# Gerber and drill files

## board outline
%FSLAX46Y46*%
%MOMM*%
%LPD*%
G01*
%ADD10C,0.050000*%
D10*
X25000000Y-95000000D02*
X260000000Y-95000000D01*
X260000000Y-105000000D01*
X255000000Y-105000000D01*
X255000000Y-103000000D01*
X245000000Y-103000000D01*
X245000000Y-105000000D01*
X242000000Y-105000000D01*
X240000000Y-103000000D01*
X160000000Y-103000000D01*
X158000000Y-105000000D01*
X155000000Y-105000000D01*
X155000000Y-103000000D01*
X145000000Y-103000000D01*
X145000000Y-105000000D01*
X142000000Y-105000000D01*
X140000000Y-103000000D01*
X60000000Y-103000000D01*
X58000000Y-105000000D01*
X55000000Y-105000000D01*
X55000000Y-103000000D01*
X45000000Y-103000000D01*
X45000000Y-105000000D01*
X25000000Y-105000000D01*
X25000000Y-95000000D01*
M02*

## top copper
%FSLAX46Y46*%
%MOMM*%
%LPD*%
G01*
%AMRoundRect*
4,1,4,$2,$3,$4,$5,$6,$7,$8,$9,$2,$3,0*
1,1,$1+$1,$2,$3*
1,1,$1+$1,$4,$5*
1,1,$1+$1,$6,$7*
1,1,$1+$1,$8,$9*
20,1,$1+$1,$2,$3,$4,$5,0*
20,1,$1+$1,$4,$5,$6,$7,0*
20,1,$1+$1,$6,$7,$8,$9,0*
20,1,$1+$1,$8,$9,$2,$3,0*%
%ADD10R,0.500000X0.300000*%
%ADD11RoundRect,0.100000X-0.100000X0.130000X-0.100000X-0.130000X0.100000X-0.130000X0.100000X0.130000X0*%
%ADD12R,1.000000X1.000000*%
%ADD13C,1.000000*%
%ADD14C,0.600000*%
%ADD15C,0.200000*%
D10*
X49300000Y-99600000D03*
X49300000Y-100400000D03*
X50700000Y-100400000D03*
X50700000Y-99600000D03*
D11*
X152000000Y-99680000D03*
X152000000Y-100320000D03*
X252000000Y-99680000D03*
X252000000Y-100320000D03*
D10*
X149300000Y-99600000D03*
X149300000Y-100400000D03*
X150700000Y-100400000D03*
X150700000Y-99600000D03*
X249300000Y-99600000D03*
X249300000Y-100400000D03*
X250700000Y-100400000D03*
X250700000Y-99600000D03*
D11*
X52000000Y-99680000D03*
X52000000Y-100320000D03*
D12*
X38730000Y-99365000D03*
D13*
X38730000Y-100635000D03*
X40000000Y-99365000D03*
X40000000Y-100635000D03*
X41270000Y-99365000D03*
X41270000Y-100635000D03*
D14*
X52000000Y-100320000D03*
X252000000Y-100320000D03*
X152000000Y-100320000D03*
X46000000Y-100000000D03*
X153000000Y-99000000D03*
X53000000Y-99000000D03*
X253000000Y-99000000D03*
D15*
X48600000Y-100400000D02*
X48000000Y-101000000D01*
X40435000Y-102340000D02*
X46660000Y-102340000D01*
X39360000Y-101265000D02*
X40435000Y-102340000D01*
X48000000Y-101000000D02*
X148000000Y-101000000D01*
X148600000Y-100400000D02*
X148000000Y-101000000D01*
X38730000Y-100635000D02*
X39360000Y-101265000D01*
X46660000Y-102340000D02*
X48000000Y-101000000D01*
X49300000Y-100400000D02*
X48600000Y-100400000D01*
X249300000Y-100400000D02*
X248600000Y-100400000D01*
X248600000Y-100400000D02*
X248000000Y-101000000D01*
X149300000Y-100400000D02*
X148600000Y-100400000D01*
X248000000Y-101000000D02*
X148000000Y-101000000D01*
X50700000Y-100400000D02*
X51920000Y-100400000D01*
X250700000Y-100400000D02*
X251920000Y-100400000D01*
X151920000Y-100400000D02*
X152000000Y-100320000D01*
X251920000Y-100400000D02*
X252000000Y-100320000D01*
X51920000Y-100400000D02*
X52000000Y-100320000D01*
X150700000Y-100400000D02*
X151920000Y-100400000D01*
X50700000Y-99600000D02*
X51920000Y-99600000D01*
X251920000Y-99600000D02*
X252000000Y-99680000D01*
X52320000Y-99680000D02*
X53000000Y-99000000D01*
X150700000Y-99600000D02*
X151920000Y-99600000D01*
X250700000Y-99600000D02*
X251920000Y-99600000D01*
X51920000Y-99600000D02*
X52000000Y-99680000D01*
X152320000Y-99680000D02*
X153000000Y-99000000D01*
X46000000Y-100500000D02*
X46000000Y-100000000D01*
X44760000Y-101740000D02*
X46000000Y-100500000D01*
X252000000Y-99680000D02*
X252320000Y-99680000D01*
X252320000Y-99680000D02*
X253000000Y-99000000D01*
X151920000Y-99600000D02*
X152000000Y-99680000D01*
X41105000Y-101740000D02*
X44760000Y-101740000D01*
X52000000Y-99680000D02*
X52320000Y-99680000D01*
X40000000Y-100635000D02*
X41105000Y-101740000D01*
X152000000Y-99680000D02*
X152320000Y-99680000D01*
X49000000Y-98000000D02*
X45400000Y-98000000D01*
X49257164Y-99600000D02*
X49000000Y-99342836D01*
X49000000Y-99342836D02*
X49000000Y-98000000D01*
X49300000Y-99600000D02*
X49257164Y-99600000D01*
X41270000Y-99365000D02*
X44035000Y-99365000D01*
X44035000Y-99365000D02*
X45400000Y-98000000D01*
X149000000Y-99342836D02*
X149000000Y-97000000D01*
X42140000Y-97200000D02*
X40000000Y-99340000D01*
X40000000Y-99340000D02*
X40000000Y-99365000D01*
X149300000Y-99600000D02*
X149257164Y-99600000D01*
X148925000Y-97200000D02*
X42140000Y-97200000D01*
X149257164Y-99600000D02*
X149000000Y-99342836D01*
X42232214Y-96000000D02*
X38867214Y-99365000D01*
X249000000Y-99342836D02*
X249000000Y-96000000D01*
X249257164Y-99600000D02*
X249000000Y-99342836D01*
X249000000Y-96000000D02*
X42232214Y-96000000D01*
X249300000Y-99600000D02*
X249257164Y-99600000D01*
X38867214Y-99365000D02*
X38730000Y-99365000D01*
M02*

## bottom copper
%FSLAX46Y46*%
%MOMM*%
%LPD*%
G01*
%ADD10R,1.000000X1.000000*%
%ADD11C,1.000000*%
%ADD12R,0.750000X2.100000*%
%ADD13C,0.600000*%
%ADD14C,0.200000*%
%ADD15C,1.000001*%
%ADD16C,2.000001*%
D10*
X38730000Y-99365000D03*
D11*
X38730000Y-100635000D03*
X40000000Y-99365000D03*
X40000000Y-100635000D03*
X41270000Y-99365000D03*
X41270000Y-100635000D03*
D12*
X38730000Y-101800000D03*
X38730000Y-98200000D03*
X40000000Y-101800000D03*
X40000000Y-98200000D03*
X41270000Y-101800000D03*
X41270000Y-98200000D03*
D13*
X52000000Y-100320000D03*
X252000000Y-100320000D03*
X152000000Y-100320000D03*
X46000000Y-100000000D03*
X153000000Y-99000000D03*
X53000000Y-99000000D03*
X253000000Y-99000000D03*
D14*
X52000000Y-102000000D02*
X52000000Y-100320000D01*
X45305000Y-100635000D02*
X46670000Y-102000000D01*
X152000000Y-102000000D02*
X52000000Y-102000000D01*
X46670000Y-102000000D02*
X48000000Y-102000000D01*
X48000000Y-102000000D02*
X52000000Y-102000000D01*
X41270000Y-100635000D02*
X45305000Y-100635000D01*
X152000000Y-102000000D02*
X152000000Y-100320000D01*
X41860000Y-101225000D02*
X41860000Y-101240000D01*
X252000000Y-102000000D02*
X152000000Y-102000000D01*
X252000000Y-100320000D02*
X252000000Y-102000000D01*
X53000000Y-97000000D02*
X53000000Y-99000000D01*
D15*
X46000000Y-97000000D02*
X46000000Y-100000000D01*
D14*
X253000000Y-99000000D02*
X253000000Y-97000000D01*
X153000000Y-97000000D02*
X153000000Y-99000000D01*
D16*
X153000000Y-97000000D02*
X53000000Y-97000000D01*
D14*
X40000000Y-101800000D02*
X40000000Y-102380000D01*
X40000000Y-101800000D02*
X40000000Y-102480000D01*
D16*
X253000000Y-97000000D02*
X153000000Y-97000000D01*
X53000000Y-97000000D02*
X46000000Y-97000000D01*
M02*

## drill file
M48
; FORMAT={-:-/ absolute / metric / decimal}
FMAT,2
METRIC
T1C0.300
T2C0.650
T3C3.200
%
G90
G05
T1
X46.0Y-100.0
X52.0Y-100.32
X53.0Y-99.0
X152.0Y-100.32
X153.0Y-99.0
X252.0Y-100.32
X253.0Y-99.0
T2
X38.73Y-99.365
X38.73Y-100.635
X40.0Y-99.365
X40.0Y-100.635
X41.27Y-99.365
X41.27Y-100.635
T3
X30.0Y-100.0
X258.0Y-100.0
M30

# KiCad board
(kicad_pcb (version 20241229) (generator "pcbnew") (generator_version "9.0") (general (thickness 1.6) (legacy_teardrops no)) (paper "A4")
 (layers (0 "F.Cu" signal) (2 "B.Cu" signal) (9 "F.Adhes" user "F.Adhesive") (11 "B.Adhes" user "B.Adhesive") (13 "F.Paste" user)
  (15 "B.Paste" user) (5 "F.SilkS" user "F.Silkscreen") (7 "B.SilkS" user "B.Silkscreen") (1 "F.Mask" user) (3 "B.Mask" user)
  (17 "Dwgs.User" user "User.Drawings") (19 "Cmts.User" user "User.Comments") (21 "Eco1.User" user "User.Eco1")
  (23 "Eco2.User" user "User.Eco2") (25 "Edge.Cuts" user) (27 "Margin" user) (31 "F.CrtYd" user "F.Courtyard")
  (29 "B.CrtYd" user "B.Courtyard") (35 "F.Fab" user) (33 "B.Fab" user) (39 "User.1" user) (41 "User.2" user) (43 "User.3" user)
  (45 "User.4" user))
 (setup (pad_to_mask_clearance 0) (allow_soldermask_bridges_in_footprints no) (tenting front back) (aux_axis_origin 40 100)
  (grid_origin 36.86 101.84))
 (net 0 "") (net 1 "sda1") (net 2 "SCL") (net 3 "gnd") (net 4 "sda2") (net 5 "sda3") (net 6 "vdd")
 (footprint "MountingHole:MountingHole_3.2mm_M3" (layer "F.Cu") (at 258 100)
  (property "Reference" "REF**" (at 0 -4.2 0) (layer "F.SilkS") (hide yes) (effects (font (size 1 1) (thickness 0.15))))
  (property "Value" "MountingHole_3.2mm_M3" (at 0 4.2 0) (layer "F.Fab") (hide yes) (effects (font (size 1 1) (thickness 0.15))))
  (pad "" np_thru_hole circle (at 0 0) (size 3.2 3.2) (drill 3.2) (layers "*.Cu" "*.Mask")))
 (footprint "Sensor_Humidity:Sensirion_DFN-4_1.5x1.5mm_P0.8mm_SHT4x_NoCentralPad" (layer "F.Cu") (at 50 100)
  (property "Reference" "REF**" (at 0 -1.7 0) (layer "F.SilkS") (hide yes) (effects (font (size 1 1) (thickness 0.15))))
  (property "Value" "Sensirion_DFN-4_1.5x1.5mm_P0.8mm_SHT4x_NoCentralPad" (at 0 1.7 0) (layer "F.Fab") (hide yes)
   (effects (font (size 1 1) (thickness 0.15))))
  (pad "1" smd rect (at -0.7 -0.4) (size 0.5 0.3) (layers "F.Cu" "F.Mask" "F.Paste") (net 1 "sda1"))
  (pad "2" smd rect (at -0.7 0.4) (size 0.5 0.3) (layers "F.Cu" "F.Mask" "F.Paste") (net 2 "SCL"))
  (pad "3" smd rect (at 0.7 0.4) (size 0.5 0.3) (layers "F.Cu" "F.Mask" "F.Paste"))
  (pad "4" smd rect (at 0.7 -0.4) (size 0.5 0.3) (layers "F.Cu" "F.Mask" "F.Paste") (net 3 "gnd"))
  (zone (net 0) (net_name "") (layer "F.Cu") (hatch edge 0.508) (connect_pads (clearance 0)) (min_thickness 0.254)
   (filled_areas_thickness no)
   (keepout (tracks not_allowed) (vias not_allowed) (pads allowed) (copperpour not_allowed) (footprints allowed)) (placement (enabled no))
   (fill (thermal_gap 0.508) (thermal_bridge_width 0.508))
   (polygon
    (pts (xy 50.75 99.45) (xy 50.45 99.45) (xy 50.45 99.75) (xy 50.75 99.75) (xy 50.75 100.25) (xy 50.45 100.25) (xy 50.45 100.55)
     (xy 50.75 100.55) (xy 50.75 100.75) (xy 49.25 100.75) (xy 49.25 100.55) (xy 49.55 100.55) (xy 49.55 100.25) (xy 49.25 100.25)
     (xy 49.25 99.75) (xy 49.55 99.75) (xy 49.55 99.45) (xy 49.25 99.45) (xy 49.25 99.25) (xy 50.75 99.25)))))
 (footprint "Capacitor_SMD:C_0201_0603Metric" (layer "F.Cu") (at 152 100 -90)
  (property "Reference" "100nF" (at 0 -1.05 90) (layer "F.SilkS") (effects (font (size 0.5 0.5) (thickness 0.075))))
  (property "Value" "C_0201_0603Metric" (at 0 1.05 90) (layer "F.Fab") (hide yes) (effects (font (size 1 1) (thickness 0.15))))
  (pad "" smd roundrect (at -0.345 0 270) (size 0.318 0.36) (layers "F.Paste") (roundrect_rratio 0.25))
  (pad "" smd roundrect (at 0.345 0 270) (size 0.318 0.36) (layers "F.Paste") (roundrect_rratio 0.25))
  (pad "1" smd roundrect (at -0.32 0 270) (size 0.46 0.4) (layers "F.Cu" "F.Mask") (roundrect_rratio 0.25))
  (pad "2" smd roundrect (at 0.32 0 270) (size 0.46 0.4) (layers "F.Cu" "F.Mask") (roundrect_rratio 0.25)))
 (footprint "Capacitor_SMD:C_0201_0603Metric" (layer "F.Cu") (at 252 100 -90)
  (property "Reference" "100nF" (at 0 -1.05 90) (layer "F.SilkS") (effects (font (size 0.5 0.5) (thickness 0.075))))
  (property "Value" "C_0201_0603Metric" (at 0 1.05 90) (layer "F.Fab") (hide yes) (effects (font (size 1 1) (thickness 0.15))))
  (pad "" smd roundrect (at -0.345 0 270) (size 0.318 0.36) (layers "F.Paste") (roundrect_rratio 0.25))
  (pad "" smd roundrect (at 0.345 0 270) (size 0.318 0.36) (layers "F.Paste") (roundrect_rratio 0.25))
  (pad "1" smd roundrect (at -0.32 0 270) (size 0.46 0.4) (layers "F.Cu" "F.Mask") (roundrect_rratio 0.25))
  (pad "2" smd roundrect (at 0.32 0 270) (size 0.46 0.4) (layers "F.Cu" "F.Mask") (roundrect_rratio 0.25)))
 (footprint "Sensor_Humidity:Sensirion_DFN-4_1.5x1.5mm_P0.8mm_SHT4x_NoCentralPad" (layer "F.Cu") (at 150 100)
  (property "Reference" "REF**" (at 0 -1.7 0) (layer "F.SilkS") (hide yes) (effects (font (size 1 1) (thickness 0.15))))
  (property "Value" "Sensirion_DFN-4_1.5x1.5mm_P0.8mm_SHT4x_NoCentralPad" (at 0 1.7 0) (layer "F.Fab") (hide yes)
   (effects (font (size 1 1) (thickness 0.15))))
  (pad "1" smd rect (at -0.7 -0.4) (size 0.5 0.3) (layers "F.Cu" "F.Mask" "F.Paste") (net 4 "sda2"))
  (pad "2" smd rect (at -0.7 0.4) (size 0.5 0.3) (layers "F.Cu" "F.Mask" "F.Paste") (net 2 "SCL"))
  (pad "3" smd rect (at 0.7 0.4) (size 0.5 0.3) (layers "F.Cu" "F.Mask" "F.Paste"))
  (pad "4" smd rect (at 0.7 -0.4) (size 0.5 0.3) (layers "F.Cu" "F.Mask" "F.Paste"))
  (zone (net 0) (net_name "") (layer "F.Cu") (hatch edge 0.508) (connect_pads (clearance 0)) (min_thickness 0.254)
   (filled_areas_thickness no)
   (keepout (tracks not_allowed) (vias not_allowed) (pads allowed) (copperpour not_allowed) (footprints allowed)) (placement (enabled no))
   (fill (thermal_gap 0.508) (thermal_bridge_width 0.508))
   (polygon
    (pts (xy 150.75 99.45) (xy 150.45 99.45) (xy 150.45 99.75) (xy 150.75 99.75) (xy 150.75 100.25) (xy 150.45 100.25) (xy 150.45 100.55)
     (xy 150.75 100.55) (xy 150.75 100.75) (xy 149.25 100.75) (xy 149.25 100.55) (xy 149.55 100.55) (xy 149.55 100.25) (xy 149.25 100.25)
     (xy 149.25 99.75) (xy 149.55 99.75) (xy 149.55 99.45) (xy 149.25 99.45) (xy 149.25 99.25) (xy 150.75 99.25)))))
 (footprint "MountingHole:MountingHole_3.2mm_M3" (layer "F.Cu") (at 30 100)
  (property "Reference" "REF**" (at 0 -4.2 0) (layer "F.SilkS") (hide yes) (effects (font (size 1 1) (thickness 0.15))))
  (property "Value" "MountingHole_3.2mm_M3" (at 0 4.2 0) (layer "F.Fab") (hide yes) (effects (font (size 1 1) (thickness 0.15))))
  (pad "" np_thru_hole circle (at 0 0) (size 3.2 3.2) (drill 3.2) (layers "*.Cu" "*.Mask")))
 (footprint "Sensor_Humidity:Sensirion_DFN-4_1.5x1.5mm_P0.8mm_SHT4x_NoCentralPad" (layer "F.Cu") (at 250 100)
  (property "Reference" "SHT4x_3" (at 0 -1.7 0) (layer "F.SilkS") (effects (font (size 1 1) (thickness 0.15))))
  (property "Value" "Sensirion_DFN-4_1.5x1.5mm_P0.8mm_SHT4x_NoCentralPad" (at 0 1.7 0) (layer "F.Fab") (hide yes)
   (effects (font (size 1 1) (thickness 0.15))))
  (pad "1" smd rect (at -0.7 -0.4) (size 0.5 0.3) (layers "F.Cu" "F.Mask" "F.Paste") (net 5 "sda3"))
  (pad "2" smd rect (at -0.7 0.4) (size 0.5 0.3) (layers "F.Cu" "F.Mask" "F.Paste") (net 2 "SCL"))
  (pad "3" smd rect (at 0.7 0.4) (size 0.5 0.3) (layers "F.Cu" "F.Mask" "F.Paste") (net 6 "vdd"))
  (pad "4" smd rect (at 0.7 -0.4) (size 0.5 0.3) (layers "F.Cu" "F.Mask" "F.Paste"))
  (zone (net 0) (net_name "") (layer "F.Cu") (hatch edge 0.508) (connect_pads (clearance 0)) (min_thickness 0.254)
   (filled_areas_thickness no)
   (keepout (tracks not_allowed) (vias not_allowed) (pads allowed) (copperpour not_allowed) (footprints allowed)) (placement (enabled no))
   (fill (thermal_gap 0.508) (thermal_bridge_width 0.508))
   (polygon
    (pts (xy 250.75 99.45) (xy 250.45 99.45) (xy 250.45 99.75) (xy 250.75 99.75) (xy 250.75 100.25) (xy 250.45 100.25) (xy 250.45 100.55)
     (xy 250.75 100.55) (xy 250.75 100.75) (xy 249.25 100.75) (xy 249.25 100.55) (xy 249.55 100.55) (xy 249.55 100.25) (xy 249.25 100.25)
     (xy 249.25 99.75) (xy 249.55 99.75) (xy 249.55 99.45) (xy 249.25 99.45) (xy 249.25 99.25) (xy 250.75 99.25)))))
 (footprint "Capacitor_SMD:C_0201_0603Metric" (layer "F.Cu") (at 52 100 -90)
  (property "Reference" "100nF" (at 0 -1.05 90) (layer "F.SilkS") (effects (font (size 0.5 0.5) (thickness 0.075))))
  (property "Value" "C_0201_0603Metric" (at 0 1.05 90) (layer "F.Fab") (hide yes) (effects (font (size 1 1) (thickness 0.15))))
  (pad "" smd roundrect (at -0.345 0 270) (size 0.318 0.36) (layers "F.Paste") (roundrect_rratio 0.25))
  (pad "" smd roundrect (at 0.345 0 270) (size 0.318 0.36) (layers "F.Paste") (roundrect_rratio 0.25))
  (pad "1" smd roundrect (at -0.32 0 270) (size 0.46 0.4) (layers "F.Cu" "F.Mask") (roundrect_rratio 0.25))
  (pad "2" smd roundrect (at 0.32 0 270) (size 0.46 0.4) (layers "F.Cu" "F.Mask") (roundrect_rratio 0.25)))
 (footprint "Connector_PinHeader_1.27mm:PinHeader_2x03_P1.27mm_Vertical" (layer "B.Cu") (at 38.73 99.365 -90)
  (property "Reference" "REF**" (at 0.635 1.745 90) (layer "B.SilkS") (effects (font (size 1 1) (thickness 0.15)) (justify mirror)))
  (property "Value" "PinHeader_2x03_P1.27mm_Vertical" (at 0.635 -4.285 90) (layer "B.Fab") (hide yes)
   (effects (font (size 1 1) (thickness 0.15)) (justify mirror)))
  (pad "1" thru_hole rect (at 0 0 270) (size 1 1) (drill 0.65) (layers "*.Cu" "*.Mask") (remove_unused_layers no) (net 5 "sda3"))
  (pad "2" thru_hole circle (at 1.27 0 270) (size 1 1) (drill 0.65) (layers "*.Cu" "*.Mask") (remove_unused_layers no) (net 2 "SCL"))
  (pad "3" thru_hole circle (at 0 -1.27 270) (size 1 1) (drill 0.65) (layers "*.Cu" "*.Mask") (remove_unused_layers no) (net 4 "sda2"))
  (pad "4" thru_hole circle (at 1.27 -1.27 270) (size 1 1) (drill 0.65) (layers "*.Cu" "*.Mask") (remove_unused_layers no) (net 3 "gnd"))
  (pad "5" thru_hole circle (at 0 -2.54 270) (size 1 1) (drill 0.65) (layers "*.Cu" "*.Mask") (remove_unused_layers no) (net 1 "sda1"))
  (pad "6" thru_hole circle (at 1.27 -2.54 270) (size 1 1) (drill 0.65) (layers "*.Cu" "*.Mask") (remove_unused_layers no) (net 6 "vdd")))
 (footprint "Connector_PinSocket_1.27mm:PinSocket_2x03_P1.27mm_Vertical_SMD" (layer "B.Cu") (at 40 100 -90)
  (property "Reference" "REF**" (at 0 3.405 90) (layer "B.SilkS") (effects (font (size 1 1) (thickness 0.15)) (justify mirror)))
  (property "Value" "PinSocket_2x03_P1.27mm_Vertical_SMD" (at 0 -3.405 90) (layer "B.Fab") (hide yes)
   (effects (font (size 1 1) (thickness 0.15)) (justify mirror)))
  (pad "1" smd rect (at 1.8 1.27 270) (size 2.1 0.75) (layers "B.Cu" "B.Mask" "B.Paste") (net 2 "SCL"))
  (pad "2" smd rect (at -1.8 1.27 270) (size 2.1 0.75) (layers "B.Cu" "B.Mask" "B.Paste") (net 5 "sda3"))
  (pad "3" smd rect (at 1.8 0 270) (size 2.1 0.75) (layers "B.Cu" "B.Mask" "B.Paste") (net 3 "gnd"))
  (pad "4" smd rect (at -1.8 0 270) (size 2.1 0.75) (layers "B.Cu" "B.Mask" "B.Paste") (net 4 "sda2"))
  (pad "5" smd rect (at 1.8 -1.27 270) (size 2.1 0.75) (layers "B.Cu" "B.Mask" "B.Paste") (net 6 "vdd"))
  (pad "6" smd rect (at -1.8 -1.27 270) (size 2.1 0.75) (layers "B.Cu" "B.Mask" "B.Paste") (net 1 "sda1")))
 (gr_poly
  (pts (xy 25 95) (xy 260 95) (xy 260 105) (xy 255 105) (xy 255 103) (xy 245 103) (xy 245 105) (xy 242 105) (xy 240 103) (xy 160 103)
   (xy 158 105) (xy 155 105) (xy 155 103) (xy 145 103) (xy 145 105) (xy 142 105) (xy 140 103) (xy 60 103) (xy 58 105) (xy 55 105)
   (xy 55 103) (xy 45 103) (xy 45 105) (xy 25 105))
  (stroke (width 0.05) (type solid)) (fill no) (layer "Edge.Cuts"))
 (segment (start 48.6 100.4) (end 48 101) (width 0.2) (layer "F.Cu") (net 2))
 (segment (start 40.435 102.34) (end 46.66 102.34) (width 0.2) (layer "F.Cu") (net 2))
 (segment (start 39.36 101.265) (end 40.435 102.34) (width 0.2) (layer "F.Cu") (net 2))
 (segment (start 48 101) (end 148 101) (width 0.2) (layer "F.Cu") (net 2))
 (segment (start 148.6 100.4) (end 148 101) (width 0.2) (layer "F.Cu") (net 2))
 (segment (start 38.73 100.635) (end 39.36 101.265) (width 0.2) (layer "F.Cu") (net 2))
 (segment (start 46.66 102.34) (end 48 101) (width 0.2) (layer "F.Cu") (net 2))
 (segment (start 49.3 100.4) (end 48.6 100.4) (width 0.2) (layer "F.Cu") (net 2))
 (segment (start 249.3 100.4) (end 248.6 100.4) (width 0.2) (layer "F.Cu") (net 2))
 (segment (start 248.6 100.4) (end 248 101) (width 0.2) (layer "F.Cu") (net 2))
 (segment (start 149.3 100.4) (end 148.6 100.4) (width 0.2) (layer "F.Cu") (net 2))
 (segment (start 248 101) (end 148 101) (width 0.2) (layer "F.Cu") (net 2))
 (segment (start 50.7 100.4) (end 51.92 100.4) (width 0.2) (layer "F.Cu") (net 6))
 (segment (start 250.7 100.4) (end 251.92 100.4) (width 0.2) (layer "F.Cu") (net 6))
 (segment (start 151.92 100.4) (end 152 100.32) (width 0.2) (layer "F.Cu") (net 6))
 (segment (start 251.92 100.4) (end 252 100.32) (width 0.2) (layer "F.Cu") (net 6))
 (segment (start 51.92 100.4) (end 52 100.32) (width 0.2) (layer "F.Cu") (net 6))
 (segment (start 150.7 100.4) (end 151.92 100.4) (width 0.2) (layer "F.Cu") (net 6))
 (via blind (at 52 100.32) (size 0.6) (drill 0.3) (layers "F.Cu" "B.Cu") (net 6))
 (via blind (at 252 100.32) (size 0.6) (drill 0.3) (layers "F.Cu" "B.Cu") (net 6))
 (via blind (at 152 100.32) (size 0.6) (drill 0.3) (layers "F.Cu" "B.Cu") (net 6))
 (segment (start 52 102) (end 52 100.32) (width 0.2) (layer "B.Cu") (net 6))
 (segment (start 45.305 100.635) (end 46.67 102) (width 0.2) (layer "B.Cu") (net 6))
 (segment (start 152 102) (end 52 102) (width 0.2) (layer "B.Cu") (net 6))
 (segment (start 46.67 102) (end 48 102) (width 0.2) (layer "B.Cu") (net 6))
 (segment (start 48 102) (end 52 102) (width 0.2) (layer "B.Cu") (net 6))
 (segment (start 41.27 100.635) (end 45.305 100.635) (width 0.2) (layer "B.Cu") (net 6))
 (segment (start 152 102) (end 152 100.32) (width 0.2) (layer "B.Cu") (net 6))
 (segment (start 41.86 101.225) (end 41.86 101.24) (width 0.2) (layer "B.Cu") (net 6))
 (segment (start 252 102) (end 152 102) (width 0.2) (layer "B.Cu") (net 6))
 (segment (start 252 100.32) (end 252 102) (width 0.2) (layer "B.Cu") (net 6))
 (segment (start 50.7 99.6) (end 51.92 99.6) (width 0.2) (layer "F.Cu") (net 3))
 (segment (start 251.92 99.6) (end 252 99.68) (width 0.2) (layer "F.Cu") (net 3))
 (segment (start 52.32 99.68) (end 53 99) (width 0.2) (layer "F.Cu") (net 3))
 (segment (start 150.7 99.6) (end 151.92 99.6) (width 0.2) (layer "F.Cu") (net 3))
 (segment (start 250.7 99.6) (end 251.92 99.6) (width 0.2) (layer "F.Cu") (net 3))
 (segment (start 51.92 99.6) (end 52 99.68) (width 0.2) (layer "F.Cu") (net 3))
 (segment (start 152.32 99.68) (end 153 99) (width 0.2) (layer "F.Cu") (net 3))
 (segment (start 46 100.5) (end 46 100) (width 0.2) (layer "F.Cu") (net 3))
 (segment (start 44.76 101.74) (end 46 100.5) (width 0.2) (layer "F.Cu") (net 3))
 (segment (start 252 99.68) (end 252.32 99.68) (width 0.2) (layer "F.Cu") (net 3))
 (segment (start 252.32 99.68) (end 253 99) (width 0.2) (layer "F.Cu") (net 3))
 (segment (start 151.92 99.6) (end 152 99.68) (width 0.2) (layer "F.Cu") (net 3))
 (segment (start 41.105 101.74) (end 44.76 101.74) (width 0.2) (layer "F.Cu") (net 3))
 (segment (start 52 99.68) (end 52.32 99.68) (width 0.2) (layer "F.Cu") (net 3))
 (segment (start 40 100.635) (end 41.105 101.74) (width 0.2) (layer "F.Cu") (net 3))
 (segment (start 152 99.68) (end 152.32 99.68) (width 0.2) (layer "F.Cu") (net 3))
 (via (at 46 100) (size 0.6) (drill 0.3) (layers "F.Cu" "B.Cu") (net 3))
 (via blind (at 153 99) (size 0.6) (drill 0.3) (layers "F.Cu" "B.Cu") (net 3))
 (via blind (at 53 99) (size 0.6) (drill 0.3) (layers "F.Cu" "B.Cu") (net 3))
 (via blind (at 253 99) (size 0.6) (drill 0.3) (layers "F.Cu" "B.Cu") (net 3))
 (segment (start 53 97) (end 53 99) (width 0.2) (layer "B.Cu") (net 3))
 (segment (start 46 97) (end 46 100) (width 1.000001) (layer "B.Cu") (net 3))
 (segment (start 253 99) (end 253 97) (width 0.2) (layer "B.Cu") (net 3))
 (segment (start 153 97) (end 153 99) (width 0.2) (layer "B.Cu") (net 3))
 (segment (start 153 97) (end 53 97) (width 2.000001) (layer "B.Cu") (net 3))
 (segment (start 40 101.8) (end 40 102.38) (width 0.2) (layer "B.Cu") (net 3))
 (segment (start 40 101.8) (end 40 102.48) (width 0.2) (layer "B.Cu") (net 3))
 (segment (start 253 97) (end 153 97) (width 2.000001) (layer "B.Cu") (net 3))
 (segment (start 53 97) (end 46 97) (width 2.000001) (layer "B.Cu") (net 3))
 (segment (start 49 98) (end 45.4 98) (width 0.2) (layer "F.Cu") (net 1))
 (segment (start 49.257164 99.6) (end 49 99.342836) (width 0.2) (layer "F.Cu") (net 1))
 (segment (start 49 99.342836) (end 49 98) (width 0.2) (layer "F.Cu") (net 1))
 (segment (start 49.3 99.6) (end 49.257164 99.6) (width 0.2) (layer "F.Cu") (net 1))
 (segment (start 41.27 99.365) (end 44.035 99.365) (width 0.2) (layer "F.Cu") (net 1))
 (segment (start 44.035 99.365) (end 45.4 98) (width 0.2) (layer "F.Cu") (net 1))
 (segment (start 149 99.342836) (end 149 97) (width 0.2) (layer "F.Cu") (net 4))
 (segment (start 42.14 97.2) (end 40 99.34) (width 0.2) (layer "F.Cu") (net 4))
 (segment (start 40 99.34) (end 40 99.365) (width 0.2) (layer "F.Cu") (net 4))
 (segment (start 149.3 99.6) (end 149.257164 99.6) (width 0.2) (layer "F.Cu") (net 4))
 (segment (start 148.925 97.2) (end 42.14 97.2) (width 0.2) (layer "F.Cu") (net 4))
 (segment (start 149.257164 99.6) (end 149 99.342836) (width 0.2) (layer "F.Cu") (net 4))
 (segment (start 42.232214 96) (end 38.867214 99.365) (width 0.2) (layer "F.Cu") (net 5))
 (segment (start 249 99.342836) (end 249 96) (width 0.2) (layer "F.Cu") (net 5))
 (segment (start 249.257164 99.6) (end 249 99.342836) (width 0.2) (layer "F.Cu") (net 5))
 (segment (start 249 96) (end 42.232214 96) (width 0.2) (layer "F.Cu") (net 5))
 (segment (start 249.3 99.6) (end 249.257164 99.6) (width 0.2) (layer "F.Cu") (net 5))
 (segment (start 38.867214 99.365) (end 38.73 99.365) (width 0.2) (layer "F.Cu") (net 5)))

